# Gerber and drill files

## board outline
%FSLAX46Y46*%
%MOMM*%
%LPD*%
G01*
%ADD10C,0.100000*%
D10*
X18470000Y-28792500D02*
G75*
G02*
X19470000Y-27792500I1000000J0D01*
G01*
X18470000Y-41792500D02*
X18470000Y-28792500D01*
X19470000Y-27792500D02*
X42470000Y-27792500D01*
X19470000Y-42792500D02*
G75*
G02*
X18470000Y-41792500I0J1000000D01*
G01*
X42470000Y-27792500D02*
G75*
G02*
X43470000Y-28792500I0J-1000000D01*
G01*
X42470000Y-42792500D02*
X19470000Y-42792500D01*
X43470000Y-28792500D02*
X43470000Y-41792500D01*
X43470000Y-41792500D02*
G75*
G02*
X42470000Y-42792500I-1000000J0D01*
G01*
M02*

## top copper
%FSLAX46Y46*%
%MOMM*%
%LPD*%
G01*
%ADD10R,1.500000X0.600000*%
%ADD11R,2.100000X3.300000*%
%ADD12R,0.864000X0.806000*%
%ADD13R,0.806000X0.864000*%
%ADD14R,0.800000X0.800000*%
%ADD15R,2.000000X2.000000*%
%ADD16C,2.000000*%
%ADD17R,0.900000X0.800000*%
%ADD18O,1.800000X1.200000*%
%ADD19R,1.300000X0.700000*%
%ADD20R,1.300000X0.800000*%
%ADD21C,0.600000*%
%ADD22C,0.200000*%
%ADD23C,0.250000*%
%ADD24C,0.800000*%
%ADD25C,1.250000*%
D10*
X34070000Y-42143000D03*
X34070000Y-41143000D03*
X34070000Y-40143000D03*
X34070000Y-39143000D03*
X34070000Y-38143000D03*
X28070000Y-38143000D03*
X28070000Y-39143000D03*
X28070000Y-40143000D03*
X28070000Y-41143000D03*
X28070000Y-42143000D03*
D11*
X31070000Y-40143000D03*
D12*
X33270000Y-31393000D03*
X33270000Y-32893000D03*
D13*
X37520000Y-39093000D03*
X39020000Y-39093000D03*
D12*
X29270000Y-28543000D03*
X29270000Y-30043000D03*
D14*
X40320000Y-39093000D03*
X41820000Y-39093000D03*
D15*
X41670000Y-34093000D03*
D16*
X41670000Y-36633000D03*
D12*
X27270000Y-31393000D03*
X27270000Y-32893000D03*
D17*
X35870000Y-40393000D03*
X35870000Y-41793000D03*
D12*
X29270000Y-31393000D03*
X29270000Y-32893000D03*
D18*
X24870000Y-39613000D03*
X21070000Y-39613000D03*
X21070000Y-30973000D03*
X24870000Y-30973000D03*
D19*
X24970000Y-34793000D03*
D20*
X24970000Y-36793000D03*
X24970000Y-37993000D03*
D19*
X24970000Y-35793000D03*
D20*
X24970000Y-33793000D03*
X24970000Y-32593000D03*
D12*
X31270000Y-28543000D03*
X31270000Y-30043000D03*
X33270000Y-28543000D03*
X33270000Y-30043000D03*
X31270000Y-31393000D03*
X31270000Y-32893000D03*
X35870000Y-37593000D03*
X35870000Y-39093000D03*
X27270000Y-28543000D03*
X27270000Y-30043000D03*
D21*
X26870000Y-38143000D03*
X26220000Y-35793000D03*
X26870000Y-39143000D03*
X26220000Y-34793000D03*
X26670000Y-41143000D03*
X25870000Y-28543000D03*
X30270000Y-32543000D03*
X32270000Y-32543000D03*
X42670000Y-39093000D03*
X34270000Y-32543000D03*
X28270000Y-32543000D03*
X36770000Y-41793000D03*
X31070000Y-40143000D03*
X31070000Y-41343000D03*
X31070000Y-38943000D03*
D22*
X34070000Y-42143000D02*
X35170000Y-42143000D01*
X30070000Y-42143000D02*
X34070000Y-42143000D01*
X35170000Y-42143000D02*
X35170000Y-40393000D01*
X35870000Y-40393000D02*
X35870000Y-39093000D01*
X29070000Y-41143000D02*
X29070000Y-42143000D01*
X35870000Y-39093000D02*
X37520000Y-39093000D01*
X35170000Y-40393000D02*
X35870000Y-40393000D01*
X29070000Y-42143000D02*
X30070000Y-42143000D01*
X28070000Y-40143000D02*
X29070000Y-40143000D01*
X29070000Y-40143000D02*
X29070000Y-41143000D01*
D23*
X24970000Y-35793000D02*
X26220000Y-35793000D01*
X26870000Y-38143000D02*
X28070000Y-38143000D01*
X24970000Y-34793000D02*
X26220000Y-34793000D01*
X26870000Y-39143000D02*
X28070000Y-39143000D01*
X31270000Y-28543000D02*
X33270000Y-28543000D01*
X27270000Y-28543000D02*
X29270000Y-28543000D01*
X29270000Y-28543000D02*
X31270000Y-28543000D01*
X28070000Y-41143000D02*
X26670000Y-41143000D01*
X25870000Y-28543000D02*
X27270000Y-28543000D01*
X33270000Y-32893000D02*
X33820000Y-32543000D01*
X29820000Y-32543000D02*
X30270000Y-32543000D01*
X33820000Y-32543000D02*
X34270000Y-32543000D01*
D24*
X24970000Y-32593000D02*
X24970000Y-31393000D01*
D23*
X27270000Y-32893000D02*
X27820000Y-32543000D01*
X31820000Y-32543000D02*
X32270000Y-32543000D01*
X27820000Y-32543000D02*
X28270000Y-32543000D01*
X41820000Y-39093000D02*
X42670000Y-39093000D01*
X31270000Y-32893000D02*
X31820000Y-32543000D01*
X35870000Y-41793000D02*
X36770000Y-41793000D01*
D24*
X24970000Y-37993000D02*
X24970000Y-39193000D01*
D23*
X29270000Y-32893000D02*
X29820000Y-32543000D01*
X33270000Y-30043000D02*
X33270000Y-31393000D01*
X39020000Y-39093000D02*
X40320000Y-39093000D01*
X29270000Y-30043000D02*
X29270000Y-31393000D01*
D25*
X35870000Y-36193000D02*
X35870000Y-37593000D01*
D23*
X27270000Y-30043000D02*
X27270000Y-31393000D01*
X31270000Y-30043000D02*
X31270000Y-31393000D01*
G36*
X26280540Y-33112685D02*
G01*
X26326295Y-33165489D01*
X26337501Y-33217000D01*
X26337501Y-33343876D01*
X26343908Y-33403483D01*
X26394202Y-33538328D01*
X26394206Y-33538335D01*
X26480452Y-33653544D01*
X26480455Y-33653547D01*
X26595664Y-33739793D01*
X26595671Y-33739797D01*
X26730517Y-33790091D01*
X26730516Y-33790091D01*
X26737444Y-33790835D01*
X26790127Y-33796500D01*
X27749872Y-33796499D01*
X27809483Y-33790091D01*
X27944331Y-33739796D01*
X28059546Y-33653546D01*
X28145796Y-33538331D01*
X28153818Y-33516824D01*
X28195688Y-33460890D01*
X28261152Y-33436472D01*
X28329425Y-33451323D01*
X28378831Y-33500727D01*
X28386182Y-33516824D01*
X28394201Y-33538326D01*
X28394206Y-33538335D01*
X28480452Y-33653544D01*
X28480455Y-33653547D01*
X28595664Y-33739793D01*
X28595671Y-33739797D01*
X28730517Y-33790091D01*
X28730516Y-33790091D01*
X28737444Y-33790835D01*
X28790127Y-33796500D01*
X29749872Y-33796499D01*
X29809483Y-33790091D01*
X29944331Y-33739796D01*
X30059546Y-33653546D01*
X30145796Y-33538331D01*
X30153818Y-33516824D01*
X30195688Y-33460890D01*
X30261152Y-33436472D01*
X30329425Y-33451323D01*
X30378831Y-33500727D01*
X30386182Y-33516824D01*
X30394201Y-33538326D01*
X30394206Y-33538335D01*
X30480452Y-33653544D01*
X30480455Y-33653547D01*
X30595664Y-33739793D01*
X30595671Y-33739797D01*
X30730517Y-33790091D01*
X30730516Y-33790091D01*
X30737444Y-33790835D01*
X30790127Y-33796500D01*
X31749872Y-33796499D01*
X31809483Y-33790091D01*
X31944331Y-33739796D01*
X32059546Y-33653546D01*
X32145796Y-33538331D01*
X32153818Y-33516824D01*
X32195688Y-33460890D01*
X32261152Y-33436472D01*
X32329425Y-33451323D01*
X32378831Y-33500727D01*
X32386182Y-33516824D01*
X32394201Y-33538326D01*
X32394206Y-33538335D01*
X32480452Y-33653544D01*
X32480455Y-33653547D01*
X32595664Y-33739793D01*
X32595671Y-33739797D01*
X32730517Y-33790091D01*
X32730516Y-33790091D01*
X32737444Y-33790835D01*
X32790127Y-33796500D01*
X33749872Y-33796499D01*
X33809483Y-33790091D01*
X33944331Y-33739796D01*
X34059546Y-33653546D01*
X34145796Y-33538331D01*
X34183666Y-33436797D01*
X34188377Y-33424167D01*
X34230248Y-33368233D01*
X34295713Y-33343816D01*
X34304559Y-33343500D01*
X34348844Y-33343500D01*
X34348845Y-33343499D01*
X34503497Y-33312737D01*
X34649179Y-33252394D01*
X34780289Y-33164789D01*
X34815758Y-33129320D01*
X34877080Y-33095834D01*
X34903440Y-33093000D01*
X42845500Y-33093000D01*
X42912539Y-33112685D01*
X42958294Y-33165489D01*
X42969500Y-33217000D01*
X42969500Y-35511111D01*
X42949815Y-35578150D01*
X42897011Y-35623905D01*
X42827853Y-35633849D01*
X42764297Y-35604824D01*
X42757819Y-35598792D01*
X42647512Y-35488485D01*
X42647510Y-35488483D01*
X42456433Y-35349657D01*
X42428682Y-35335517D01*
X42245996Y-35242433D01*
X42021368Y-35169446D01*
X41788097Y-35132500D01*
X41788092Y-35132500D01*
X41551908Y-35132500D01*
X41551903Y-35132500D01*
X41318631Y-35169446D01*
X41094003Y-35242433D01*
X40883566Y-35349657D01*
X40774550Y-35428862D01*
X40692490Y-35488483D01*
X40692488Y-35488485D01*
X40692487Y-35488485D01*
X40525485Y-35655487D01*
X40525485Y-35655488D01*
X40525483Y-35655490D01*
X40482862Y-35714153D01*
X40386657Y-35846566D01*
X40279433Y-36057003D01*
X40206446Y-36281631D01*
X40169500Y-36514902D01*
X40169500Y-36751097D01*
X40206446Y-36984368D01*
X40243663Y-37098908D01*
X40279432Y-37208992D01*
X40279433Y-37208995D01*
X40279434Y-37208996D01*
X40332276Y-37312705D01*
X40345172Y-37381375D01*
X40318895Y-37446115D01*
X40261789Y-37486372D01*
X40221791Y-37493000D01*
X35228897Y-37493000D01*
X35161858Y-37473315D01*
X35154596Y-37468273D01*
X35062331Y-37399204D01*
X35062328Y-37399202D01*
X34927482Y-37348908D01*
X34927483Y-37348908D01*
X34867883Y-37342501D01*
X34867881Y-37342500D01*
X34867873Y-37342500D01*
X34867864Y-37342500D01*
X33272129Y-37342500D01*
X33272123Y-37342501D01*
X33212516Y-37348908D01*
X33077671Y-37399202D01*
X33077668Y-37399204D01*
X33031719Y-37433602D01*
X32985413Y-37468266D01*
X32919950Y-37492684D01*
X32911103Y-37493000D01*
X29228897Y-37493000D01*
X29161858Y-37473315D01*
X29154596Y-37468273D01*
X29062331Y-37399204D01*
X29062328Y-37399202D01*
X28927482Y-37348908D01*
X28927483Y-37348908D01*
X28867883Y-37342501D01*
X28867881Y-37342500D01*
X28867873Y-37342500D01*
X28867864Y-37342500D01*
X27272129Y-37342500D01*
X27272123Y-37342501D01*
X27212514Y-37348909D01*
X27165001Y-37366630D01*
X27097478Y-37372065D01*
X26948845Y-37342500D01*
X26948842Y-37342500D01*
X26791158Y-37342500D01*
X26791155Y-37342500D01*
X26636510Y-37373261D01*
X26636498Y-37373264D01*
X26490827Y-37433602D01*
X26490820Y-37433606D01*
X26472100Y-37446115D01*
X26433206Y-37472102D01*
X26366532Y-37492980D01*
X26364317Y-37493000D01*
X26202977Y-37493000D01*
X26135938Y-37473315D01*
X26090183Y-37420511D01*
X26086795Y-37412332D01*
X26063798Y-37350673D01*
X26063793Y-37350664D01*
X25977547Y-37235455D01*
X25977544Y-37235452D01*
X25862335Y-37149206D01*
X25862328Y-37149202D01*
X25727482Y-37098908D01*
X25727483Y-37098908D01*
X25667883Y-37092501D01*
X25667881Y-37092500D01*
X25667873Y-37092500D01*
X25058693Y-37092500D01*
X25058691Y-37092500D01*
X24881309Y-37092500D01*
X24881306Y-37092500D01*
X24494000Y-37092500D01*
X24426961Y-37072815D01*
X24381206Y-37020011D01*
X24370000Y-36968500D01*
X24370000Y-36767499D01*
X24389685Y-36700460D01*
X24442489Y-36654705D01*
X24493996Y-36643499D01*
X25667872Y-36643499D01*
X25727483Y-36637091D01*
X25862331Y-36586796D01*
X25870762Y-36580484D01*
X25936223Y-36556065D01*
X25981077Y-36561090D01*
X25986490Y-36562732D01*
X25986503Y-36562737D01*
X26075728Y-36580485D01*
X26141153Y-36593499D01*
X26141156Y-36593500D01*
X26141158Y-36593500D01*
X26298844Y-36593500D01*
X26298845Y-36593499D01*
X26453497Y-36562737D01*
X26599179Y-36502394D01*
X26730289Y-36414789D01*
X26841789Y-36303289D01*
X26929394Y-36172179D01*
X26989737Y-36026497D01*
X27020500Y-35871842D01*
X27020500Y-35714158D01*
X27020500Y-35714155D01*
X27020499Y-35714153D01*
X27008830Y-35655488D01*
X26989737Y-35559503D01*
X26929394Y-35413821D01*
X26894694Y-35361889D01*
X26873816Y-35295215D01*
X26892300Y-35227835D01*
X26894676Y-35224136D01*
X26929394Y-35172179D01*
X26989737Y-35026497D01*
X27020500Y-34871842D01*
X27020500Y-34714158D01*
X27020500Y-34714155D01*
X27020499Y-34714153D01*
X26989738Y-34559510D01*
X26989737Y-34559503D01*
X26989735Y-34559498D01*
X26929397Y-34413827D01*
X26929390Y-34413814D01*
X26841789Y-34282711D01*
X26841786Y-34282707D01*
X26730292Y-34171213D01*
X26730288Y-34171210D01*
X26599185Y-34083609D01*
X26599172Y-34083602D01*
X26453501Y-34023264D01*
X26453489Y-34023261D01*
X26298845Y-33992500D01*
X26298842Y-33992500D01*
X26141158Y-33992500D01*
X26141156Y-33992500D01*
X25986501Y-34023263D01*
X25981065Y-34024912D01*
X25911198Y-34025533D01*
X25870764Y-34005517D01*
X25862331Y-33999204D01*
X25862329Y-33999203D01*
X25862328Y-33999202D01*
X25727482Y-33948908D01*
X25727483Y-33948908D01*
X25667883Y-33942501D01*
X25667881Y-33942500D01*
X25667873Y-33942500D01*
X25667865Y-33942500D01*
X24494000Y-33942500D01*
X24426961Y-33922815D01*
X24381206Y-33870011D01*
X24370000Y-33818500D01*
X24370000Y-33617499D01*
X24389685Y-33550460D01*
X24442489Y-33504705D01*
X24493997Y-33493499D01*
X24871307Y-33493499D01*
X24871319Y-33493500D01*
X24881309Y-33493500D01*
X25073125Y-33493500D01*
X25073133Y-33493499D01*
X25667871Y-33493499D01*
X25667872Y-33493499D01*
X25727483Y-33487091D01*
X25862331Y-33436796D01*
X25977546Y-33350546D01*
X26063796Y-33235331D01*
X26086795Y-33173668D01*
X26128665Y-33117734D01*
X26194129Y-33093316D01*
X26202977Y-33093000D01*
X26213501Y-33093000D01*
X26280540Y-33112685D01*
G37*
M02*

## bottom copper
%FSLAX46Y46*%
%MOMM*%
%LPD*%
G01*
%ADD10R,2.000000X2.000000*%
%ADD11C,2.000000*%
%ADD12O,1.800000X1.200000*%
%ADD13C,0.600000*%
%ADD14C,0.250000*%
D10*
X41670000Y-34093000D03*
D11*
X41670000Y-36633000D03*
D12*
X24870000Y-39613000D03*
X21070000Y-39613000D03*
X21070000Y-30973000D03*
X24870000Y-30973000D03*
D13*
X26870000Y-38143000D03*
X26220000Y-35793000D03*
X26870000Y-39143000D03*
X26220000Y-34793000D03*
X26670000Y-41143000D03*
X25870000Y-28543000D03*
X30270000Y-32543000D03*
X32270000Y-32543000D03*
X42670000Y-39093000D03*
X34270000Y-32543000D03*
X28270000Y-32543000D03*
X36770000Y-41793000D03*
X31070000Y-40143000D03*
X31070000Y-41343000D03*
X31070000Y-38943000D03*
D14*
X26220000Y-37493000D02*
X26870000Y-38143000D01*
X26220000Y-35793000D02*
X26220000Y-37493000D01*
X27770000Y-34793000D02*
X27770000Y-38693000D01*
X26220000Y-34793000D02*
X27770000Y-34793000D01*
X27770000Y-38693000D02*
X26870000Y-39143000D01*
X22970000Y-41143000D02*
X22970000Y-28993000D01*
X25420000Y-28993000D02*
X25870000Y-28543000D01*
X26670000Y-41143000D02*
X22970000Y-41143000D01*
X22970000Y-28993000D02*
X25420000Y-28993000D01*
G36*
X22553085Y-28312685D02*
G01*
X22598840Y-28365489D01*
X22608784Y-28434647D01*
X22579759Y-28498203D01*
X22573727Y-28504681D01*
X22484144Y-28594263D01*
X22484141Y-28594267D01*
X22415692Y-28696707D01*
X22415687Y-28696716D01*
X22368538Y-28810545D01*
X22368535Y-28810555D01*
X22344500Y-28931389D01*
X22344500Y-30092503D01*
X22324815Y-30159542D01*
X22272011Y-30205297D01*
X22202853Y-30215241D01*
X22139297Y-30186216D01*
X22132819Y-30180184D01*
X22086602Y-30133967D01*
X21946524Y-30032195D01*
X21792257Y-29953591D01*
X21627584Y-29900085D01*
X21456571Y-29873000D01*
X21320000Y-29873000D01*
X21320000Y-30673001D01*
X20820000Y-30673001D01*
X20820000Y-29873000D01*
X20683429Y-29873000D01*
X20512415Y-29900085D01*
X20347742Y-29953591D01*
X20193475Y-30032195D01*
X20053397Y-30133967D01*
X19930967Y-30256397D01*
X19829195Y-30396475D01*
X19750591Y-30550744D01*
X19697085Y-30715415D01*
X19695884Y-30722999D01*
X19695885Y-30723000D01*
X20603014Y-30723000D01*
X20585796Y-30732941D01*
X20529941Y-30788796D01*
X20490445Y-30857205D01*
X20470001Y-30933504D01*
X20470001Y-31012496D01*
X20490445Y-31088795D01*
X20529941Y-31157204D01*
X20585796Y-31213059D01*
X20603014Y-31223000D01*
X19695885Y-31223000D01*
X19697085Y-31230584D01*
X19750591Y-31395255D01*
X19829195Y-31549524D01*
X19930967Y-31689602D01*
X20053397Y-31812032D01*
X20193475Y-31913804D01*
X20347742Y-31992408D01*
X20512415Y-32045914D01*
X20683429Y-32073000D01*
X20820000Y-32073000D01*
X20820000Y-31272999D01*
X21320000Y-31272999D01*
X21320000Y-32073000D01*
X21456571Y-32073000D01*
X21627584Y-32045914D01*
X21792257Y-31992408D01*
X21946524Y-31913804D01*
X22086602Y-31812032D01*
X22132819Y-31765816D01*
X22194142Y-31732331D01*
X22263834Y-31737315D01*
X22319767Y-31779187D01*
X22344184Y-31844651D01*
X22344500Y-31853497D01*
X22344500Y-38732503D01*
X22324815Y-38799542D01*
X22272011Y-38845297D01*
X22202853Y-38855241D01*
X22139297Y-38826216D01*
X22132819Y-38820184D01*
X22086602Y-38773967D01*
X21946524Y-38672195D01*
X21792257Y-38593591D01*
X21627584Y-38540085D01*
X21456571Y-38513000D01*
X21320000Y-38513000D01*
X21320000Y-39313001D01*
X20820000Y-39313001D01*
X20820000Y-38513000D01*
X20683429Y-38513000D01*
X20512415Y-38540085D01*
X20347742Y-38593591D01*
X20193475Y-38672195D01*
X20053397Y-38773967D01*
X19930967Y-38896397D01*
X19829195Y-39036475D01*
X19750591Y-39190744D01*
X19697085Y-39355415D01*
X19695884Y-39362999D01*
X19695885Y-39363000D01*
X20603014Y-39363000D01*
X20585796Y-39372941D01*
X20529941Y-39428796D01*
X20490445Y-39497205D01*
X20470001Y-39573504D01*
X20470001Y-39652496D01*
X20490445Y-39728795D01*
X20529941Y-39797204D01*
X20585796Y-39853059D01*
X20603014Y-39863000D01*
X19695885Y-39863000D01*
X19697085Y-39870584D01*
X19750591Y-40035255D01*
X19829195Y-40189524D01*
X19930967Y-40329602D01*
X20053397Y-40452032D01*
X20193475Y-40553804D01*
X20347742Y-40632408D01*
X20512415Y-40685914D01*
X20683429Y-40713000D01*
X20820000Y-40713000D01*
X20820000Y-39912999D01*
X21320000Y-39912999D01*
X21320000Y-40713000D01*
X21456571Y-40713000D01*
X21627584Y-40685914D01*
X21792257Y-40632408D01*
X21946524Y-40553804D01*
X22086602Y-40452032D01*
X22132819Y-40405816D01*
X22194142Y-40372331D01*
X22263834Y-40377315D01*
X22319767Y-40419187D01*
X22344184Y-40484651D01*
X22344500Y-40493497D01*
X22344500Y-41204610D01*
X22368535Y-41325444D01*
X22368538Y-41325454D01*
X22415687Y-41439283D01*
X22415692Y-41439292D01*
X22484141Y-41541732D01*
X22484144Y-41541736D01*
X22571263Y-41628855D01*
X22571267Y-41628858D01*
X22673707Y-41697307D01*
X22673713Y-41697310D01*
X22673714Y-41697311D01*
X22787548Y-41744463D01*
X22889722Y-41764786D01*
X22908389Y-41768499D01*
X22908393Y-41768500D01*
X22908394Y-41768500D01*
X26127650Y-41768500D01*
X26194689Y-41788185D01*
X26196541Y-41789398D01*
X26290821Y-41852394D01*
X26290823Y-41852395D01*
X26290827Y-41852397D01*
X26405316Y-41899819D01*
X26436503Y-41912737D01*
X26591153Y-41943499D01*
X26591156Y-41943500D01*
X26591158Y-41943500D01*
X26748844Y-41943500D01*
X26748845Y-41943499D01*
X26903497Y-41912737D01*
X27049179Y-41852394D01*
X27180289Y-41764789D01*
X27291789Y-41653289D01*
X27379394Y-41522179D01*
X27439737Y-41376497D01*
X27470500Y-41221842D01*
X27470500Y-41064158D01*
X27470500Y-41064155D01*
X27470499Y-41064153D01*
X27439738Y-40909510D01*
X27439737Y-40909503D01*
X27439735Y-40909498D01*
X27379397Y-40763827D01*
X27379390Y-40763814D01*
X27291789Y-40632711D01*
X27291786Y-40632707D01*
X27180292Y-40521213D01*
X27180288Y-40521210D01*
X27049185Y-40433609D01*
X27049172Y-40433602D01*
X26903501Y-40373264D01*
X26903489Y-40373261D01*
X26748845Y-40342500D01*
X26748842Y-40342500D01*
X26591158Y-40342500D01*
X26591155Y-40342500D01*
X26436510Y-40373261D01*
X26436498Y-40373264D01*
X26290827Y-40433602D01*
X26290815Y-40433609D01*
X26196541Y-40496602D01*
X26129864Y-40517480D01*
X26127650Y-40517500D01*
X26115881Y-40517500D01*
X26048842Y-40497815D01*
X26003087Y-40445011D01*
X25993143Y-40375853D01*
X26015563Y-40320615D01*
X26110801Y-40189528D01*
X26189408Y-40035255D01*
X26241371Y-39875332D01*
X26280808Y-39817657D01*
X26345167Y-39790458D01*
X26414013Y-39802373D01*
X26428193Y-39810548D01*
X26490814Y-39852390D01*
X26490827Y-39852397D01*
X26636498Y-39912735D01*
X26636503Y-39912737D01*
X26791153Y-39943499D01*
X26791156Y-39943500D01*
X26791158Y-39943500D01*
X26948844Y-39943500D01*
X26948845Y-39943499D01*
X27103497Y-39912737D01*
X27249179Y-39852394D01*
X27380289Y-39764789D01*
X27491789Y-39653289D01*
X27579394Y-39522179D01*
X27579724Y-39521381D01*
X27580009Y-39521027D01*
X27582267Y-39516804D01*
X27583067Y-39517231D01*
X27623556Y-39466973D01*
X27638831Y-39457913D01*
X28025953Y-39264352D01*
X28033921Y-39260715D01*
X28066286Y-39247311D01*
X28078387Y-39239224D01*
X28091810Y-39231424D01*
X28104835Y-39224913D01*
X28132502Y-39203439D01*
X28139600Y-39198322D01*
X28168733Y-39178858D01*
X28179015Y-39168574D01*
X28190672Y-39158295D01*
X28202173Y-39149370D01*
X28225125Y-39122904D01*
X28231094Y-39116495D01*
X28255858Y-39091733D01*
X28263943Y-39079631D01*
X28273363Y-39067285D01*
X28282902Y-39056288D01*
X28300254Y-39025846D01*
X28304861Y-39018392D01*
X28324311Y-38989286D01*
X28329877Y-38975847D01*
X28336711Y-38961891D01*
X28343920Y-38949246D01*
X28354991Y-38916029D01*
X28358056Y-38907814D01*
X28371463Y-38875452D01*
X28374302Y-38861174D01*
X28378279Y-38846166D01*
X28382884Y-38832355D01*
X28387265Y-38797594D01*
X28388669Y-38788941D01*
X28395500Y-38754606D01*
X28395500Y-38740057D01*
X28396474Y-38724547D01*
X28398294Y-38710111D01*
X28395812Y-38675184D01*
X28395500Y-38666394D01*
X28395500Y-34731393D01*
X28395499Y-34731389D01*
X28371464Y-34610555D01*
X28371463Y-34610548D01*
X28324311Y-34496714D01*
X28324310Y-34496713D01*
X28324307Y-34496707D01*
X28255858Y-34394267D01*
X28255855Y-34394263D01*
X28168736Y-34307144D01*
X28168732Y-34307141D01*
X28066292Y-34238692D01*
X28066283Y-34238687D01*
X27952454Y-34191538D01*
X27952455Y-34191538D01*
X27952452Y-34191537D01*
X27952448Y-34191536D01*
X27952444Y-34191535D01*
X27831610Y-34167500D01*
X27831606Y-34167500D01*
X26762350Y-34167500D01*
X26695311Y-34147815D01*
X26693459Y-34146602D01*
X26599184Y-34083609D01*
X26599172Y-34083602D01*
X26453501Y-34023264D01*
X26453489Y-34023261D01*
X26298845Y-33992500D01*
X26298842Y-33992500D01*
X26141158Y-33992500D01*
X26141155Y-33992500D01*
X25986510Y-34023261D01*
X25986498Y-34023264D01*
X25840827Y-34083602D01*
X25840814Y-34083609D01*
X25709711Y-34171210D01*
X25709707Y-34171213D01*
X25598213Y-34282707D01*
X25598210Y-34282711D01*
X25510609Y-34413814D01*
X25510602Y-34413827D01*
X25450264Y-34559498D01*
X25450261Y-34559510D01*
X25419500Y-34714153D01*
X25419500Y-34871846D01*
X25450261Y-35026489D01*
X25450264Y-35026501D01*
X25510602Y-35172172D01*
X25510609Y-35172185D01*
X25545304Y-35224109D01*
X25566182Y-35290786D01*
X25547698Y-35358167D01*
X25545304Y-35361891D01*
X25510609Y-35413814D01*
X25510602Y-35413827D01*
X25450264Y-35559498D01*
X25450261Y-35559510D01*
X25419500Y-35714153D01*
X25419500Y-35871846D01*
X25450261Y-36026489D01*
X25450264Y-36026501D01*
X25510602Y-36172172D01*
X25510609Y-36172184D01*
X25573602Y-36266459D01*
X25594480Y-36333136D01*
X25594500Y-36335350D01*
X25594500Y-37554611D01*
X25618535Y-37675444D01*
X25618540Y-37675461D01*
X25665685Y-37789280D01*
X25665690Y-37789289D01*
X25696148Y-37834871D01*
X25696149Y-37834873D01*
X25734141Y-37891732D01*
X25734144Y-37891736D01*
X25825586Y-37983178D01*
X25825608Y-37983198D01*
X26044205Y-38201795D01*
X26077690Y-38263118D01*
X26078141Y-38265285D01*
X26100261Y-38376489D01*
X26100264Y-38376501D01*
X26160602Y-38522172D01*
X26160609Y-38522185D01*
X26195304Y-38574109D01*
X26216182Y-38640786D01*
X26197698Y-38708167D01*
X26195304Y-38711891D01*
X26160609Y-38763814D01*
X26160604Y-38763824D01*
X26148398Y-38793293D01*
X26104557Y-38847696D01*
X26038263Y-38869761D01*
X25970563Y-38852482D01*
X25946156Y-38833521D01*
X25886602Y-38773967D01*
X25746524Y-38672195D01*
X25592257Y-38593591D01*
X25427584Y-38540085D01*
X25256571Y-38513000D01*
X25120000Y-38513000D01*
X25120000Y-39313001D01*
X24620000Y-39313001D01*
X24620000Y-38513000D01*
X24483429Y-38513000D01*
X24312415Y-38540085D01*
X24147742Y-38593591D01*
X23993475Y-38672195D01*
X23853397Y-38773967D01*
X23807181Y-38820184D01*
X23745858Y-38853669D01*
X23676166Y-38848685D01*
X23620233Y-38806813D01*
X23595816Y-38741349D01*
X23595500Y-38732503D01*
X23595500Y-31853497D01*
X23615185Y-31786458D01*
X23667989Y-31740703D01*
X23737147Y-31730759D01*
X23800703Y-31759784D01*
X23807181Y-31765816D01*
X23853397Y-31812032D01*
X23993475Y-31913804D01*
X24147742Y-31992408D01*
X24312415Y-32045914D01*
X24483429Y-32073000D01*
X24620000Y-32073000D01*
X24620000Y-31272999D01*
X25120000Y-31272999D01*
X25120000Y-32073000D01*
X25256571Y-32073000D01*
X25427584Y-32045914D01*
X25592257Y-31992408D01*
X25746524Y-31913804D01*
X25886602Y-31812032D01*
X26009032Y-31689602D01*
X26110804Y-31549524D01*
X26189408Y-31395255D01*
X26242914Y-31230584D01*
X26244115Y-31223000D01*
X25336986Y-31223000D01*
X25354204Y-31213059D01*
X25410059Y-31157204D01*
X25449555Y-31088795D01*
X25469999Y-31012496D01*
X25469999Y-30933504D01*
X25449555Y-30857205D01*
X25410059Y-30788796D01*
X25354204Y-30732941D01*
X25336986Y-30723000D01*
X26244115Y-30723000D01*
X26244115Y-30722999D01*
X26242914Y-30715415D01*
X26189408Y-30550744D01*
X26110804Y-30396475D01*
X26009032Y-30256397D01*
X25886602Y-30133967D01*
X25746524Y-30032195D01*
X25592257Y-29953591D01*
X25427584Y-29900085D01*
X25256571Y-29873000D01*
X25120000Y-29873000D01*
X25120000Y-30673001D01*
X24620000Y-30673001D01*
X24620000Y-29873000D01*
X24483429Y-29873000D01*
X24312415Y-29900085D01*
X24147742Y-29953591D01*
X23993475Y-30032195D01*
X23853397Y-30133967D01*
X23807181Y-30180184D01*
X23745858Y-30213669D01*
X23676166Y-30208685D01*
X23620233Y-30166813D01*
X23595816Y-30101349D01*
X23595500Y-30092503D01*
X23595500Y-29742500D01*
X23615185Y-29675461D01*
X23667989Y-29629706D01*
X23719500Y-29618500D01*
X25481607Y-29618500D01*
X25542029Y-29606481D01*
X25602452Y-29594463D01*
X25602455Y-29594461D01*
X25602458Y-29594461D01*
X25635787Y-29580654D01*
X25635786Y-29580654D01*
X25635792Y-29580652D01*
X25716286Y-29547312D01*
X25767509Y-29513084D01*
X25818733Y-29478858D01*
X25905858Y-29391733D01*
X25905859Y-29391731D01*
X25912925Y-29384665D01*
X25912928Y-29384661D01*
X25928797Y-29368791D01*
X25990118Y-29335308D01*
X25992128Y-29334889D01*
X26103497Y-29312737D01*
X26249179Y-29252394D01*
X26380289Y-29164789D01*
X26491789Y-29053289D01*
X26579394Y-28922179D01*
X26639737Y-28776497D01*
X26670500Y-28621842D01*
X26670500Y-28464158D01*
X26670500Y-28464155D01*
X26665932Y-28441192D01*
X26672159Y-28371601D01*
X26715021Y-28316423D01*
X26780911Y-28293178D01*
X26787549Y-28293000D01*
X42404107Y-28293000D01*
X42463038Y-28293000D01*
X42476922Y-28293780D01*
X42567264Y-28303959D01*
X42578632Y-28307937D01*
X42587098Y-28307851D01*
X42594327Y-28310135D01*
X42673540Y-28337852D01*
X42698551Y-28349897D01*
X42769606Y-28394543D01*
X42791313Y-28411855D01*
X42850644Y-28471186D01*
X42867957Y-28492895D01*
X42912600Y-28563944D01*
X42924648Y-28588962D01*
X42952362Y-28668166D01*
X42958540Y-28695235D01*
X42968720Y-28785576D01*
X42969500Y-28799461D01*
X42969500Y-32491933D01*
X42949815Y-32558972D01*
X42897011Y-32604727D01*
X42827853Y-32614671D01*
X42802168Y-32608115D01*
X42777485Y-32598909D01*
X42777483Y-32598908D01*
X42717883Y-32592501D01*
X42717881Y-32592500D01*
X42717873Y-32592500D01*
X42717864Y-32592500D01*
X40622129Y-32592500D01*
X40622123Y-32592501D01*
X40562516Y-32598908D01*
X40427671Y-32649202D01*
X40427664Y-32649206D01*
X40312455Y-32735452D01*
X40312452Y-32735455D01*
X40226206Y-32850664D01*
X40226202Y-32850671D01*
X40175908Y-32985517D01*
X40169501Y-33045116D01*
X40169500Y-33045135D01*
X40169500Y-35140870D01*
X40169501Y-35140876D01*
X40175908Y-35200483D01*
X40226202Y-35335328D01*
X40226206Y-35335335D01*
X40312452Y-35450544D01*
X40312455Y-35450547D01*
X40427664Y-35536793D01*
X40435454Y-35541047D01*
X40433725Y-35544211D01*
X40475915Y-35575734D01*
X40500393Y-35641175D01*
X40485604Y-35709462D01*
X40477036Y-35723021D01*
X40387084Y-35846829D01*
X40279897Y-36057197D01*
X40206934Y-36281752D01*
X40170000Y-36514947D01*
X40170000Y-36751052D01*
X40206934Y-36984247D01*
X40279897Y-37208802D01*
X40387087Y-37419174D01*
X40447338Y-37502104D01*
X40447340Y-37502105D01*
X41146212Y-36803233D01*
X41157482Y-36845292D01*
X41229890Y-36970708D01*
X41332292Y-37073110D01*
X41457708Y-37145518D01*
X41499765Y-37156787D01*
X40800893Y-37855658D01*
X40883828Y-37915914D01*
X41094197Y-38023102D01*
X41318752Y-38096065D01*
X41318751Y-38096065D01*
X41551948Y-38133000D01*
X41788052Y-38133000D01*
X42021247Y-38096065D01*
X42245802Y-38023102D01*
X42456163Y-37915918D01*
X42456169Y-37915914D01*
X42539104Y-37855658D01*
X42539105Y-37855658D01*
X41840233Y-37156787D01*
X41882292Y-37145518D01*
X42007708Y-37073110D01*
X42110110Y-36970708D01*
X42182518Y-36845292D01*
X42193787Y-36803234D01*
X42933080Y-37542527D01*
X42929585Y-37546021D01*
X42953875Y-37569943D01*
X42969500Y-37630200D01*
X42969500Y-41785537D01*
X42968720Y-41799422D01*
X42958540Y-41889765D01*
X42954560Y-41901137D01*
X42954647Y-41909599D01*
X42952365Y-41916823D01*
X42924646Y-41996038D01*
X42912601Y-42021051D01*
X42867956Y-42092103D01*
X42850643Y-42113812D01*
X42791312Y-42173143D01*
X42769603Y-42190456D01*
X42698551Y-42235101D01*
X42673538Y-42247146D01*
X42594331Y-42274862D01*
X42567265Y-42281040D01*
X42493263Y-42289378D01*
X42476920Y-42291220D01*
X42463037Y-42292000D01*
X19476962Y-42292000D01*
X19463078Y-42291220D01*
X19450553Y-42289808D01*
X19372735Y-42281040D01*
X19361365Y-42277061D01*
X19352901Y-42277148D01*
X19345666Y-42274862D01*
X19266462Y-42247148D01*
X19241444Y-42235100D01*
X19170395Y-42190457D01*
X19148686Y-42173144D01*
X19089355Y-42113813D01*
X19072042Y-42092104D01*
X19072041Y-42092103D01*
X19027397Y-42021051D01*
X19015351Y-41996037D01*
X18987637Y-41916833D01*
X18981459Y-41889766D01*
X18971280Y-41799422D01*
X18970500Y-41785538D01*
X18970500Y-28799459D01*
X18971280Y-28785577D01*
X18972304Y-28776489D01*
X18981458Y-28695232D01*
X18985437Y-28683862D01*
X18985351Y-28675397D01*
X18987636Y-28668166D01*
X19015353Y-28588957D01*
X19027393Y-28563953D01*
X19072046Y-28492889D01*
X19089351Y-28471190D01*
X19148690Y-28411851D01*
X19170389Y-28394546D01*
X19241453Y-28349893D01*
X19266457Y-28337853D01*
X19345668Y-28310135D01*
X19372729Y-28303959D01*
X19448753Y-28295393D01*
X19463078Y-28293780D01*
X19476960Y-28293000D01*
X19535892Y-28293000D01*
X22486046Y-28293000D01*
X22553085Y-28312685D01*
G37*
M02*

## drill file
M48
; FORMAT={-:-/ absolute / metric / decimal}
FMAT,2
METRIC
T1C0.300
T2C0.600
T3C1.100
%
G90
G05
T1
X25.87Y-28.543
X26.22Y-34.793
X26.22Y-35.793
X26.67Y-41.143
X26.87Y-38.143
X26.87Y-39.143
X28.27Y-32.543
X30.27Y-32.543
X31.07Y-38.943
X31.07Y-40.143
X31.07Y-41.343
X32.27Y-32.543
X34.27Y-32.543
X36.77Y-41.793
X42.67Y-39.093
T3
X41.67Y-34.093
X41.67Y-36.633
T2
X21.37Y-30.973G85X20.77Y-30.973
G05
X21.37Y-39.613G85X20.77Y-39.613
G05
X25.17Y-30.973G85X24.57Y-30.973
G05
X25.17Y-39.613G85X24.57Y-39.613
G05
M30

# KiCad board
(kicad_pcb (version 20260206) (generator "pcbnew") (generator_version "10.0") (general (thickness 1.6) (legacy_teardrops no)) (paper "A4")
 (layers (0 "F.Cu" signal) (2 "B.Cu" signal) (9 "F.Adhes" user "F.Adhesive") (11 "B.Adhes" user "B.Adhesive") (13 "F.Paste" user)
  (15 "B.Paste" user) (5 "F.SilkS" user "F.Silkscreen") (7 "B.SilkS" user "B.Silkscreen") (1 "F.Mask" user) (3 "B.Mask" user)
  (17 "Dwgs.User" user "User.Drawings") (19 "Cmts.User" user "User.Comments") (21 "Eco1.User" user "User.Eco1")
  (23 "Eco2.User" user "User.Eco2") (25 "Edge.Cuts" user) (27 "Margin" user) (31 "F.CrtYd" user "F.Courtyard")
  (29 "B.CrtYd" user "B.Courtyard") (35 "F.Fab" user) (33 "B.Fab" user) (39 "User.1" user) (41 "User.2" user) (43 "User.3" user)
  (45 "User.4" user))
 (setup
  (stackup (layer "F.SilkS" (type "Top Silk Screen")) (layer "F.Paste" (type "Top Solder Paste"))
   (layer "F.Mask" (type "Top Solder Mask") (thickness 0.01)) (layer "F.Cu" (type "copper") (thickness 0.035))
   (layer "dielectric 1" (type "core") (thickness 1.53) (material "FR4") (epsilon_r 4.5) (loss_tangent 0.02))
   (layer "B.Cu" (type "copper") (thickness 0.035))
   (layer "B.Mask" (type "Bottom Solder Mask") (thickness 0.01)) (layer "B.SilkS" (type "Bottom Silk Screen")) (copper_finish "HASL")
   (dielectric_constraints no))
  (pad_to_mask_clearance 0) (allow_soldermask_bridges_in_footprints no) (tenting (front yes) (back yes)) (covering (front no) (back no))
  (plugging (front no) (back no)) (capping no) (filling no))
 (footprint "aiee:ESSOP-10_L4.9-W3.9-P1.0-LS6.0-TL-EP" (layer "F.Cu") (at 31.07 40.143 90)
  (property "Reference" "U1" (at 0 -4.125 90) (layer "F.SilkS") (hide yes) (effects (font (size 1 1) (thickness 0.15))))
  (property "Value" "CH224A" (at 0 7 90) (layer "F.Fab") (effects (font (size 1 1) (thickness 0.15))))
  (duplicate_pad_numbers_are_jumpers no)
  (pad "1" smd rect (at -2 3 180) (size 1.5 0.6) (layers "F.Cu" "F.Mask" "F.Paste") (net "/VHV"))
  (pad "2" smd rect (at -1 3 180) (size 1.5 0.6) (layers "F.Cu" "F.Mask" "F.Paste") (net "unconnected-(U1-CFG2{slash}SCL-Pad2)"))
  (pad "3" smd rect (at 0 3 180) (size 1.5 0.6) (layers "F.Cu" "F.Mask" "F.Paste") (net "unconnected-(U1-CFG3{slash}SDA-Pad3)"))
  (pad "4" smd rect (at 1 3 180) (size 1.5 0.6) (layers "F.Cu" "F.Mask" "F.Paste") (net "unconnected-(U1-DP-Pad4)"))
  (pad "5" smd rect (at 2 3 180) (size 1.5 0.6) (layers "F.Cu" "F.Mask" "F.Paste") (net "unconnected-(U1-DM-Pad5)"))
  (pad "6" smd rect (at 2 -3 180) (size 1.5 0.6) (layers "F.Cu" "F.Mask" "F.Paste") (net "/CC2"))
  (pad "7" smd rect (at 1 -3 180) (size 1.5 0.6) (layers "F.Cu" "F.Mask" "F.Paste") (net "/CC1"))
  (pad "8" smd rect (at 0 -3 180) (size 1.5 0.6) (layers "F.Cu" "F.Mask" "F.Paste") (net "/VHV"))
  (pad "9" smd rect (at -1 -3 180) (size 1.5 0.6) (layers "F.Cu" "F.Mask" "F.Paste") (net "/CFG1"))
  (pad "10" smd rect (at -2 -3 180) (size 1.5 0.6) (layers "F.Cu" "F.Mask" "F.Paste") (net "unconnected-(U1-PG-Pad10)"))
  (pad "11" smd rect (at 0 0 270) (size 3.3 2.1) (layers "F.Cu" "F.Mask" "F.Paste") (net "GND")))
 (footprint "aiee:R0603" (layer "F.Cu") (at 33.27 32.143 -90)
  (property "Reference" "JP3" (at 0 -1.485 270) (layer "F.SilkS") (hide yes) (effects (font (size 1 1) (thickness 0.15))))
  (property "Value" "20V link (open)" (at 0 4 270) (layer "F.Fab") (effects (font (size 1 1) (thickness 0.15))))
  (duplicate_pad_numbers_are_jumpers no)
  (pad "1" smd rect (at -0.75 0 270) (size 0.806 0.864) (layers "F.Cu" "F.Mask" "F.Paste") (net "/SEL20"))
  (pad "2" smd rect (at 0.75 0 270) (size 0.806 0.864) (layers "F.Cu" "F.Mask" "F.Paste") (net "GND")))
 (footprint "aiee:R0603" (layer "F.Cu") (at 38.27 39.093)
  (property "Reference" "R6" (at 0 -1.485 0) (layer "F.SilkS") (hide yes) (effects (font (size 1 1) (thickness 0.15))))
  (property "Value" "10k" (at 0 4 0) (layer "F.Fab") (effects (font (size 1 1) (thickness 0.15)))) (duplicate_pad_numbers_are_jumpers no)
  (pad "1" smd rect (at -0.75 0) (size 0.806 0.864) (layers "F.Cu" "F.Mask" "F.Paste") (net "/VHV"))
  (pad "2" smd rect (at 0.75 0) (size 0.806 0.864) (layers "F.Cu" "F.Mask" "F.Paste") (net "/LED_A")))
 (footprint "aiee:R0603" (layer "F.Cu") (at 29.27 29.293 -90)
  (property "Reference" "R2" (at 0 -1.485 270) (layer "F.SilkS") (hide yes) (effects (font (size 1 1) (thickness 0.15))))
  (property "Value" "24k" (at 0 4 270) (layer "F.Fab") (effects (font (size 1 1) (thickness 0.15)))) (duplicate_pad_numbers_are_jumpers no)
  (pad "1" smd rect (at -0.75 0 270) (size 0.806 0.864) (layers "F.Cu" "F.Mask" "F.Paste") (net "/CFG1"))
  (pad "2" smd rect (at 0.75 0 270) (size 0.806 0.864) (layers "F.Cu" "F.Mask" "F.Paste") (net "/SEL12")))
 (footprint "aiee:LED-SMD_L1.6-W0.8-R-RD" (layer "F.Cu") (at 41.07 39.093 180)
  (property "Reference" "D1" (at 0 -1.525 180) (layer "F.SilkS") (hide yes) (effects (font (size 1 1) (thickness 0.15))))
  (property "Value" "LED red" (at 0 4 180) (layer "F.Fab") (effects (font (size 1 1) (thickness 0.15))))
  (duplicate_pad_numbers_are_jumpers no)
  (pad "1" smd rect (at 0.75 0 180) (size 0.8 0.8) (layers "F.Cu" "F.Mask" "F.Paste") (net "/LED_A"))
  (pad "2" smd rect (at -0.75 0 180) (size 0.8 0.8) (layers "F.Cu" "F.Mask" "F.Paste") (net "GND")))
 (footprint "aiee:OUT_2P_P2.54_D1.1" (layer "F.Cu") (at 41.67 34.093)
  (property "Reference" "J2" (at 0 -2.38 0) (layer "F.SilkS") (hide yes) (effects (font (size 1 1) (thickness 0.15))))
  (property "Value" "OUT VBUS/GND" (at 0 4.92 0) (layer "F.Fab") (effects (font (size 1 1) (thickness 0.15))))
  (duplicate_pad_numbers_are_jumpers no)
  (pad "1" thru_hole rect (at 0 0) (size 2 2) (drill 1.1) (layers "*.Cu" "*.Mask") (remove_unused_layers no) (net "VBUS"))
  (pad "2" thru_hole circle (at 0 2.54) (size 2 2) (drill 1.1) (layers "*.Cu" "*.Mask") (remove_unused_layers no) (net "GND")))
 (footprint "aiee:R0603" (layer "F.Cu") (at 27.27 32.143 -90)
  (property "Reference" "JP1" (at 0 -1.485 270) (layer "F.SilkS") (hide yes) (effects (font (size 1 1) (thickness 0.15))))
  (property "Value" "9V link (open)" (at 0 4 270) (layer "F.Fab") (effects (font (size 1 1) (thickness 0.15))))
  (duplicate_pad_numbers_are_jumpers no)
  (pad "1" smd rect (at -0.75 0 270) (size 0.806 0.864) (layers "F.Cu" "F.Mask" "F.Paste") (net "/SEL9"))
  (pad "2" smd rect (at 0.75 0 270) (size 0.806 0.864) (layers "F.Cu" "F.Mask" "F.Paste") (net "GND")))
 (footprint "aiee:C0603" (layer "F.Cu") (at 35.87 41.093 -90)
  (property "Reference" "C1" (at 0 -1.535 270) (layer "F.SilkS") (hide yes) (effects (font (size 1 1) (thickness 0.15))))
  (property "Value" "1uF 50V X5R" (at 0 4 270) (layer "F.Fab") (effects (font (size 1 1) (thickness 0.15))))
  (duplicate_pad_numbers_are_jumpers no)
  (pad "1" smd rect (at -0.7 0 270) (size 0.8 0.9) (layers "F.Cu" "F.Mask" "F.Paste") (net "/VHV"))
  (pad "2" smd rect (at 0.7 0 270) (size 0.8 0.9) (layers "F.Cu" "F.Mask" "F.Paste") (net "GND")))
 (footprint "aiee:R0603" (layer "F.Cu") (at 29.27 32.143 -90)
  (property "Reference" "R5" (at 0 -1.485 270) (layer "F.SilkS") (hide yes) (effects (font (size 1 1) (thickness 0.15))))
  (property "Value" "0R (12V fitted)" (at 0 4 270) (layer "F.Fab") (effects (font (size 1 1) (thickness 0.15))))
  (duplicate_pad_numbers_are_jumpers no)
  (pad "1" smd rect (at -0.75 0 270) (size 0.806 0.864) (layers "F.Cu" "F.Mask" "F.Paste") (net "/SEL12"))
  (pad "2" smd rect (at 0.75 0 270) (size 0.806 0.864) (layers "F.Cu" "F.Mask" "F.Paste") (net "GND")))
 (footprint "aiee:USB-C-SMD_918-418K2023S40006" (layer "F.Cu") (at 23.02 35.293 -90)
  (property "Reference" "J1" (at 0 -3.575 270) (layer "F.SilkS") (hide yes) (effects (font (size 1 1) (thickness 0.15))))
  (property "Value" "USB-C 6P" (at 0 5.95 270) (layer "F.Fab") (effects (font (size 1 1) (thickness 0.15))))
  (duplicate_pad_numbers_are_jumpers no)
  (pad "1" thru_hole oval (at 4.32 -1.85 270) (size 1.2 1.8) (drill oval 0.599998 1.199998) (layers "*.Cu" "*.Mask")
   (remove_unused_layers no) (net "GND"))
  (pad "2" thru_hole oval (at 4.32 1.95 270) (size 1.2 1.8) (drill oval 0.599998 1.199998) (layers "*.Cu" "*.Mask")
   (remove_unused_layers no) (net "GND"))
  (pad "3" thru_hole oval (at -4.32 1.95 270) (size 1.2 1.8) (drill oval 0.599998 1.199998) (layers "*.Cu" "*.Mask")
   (remove_unused_layers no) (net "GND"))
  (pad "4" thru_hole oval (at -4.32 -1.85 270) (size 1.2 1.8) (drill oval 0.599998 1.199998) (layers "*.Cu" "*.Mask")
   (remove_unused_layers no) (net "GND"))
  (pad "A5" smd rect (at -0.5 -1.95 270) (size 0.7 1.3) (layers "F.Cu" "F.Mask" "F.Paste") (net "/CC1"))
  (pad "A9" smd rect (at 1.5 -1.95 270) (size 0.8 1.3) (layers "F.Cu" "F.Mask" "F.Paste") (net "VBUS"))
  (pad "A12" smd rect (at 2.7 -1.95 270) (size 0.8 1.3) (layers "F.Cu" "F.Mask" "F.Paste") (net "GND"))
  (pad "B5" smd rect (at 0.5 -1.95 270) (size 0.7 1.3) (layers "F.Cu" "F.Mask" "F.Paste") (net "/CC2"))
  (pad "B9" smd rect (at -1.5 -1.95 270) (size 0.8 1.3) (layers "F.Cu" "F.Mask" "F.Paste") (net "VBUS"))
  (pad "B12" smd rect (at -2.7 -1.95 270) (size 0.8 1.3) (layers "F.Cu" "F.Mask" "F.Paste") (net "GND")))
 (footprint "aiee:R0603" (layer "F.Cu") (at 31.27 29.293 -90)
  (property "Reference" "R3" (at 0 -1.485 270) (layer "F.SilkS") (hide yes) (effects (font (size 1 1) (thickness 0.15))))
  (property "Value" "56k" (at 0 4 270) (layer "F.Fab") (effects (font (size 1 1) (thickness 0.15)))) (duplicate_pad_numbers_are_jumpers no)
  (pad "1" smd rect (at -0.75 0 270) (size 0.806 0.864) (layers "F.Cu" "F.Mask" "F.Paste") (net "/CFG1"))
  (pad "2" smd rect (at 0.75 0 270) (size 0.806 0.864) (layers "F.Cu" "F.Mask" "F.Paste") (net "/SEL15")))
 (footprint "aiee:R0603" (layer "F.Cu") (at 33.27 29.293 -90)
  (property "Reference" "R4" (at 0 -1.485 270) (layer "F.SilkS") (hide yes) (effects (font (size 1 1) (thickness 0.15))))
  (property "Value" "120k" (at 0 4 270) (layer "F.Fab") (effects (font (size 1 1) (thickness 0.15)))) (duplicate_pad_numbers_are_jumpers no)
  (pad "1" smd rect (at -0.75 0 270) (size 0.806 0.864) (layers "F.Cu" "F.Mask" "F.Paste") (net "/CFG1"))
  (pad "2" smd rect (at 0.75 0 270) (size 0.806 0.864) (layers "F.Cu" "F.Mask" "F.Paste") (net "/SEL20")))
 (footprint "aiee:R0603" (layer "F.Cu") (at 31.27 32.143 -90)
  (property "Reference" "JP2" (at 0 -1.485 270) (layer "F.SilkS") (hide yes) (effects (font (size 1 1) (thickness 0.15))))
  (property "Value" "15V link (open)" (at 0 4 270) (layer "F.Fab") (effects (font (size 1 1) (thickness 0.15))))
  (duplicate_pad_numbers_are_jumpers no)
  (pad "1" smd rect (at -0.75 0 270) (size 0.806 0.864) (layers "F.Cu" "F.Mask" "F.Paste") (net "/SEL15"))
  (pad "2" smd rect (at 0.75 0 270) (size 0.806 0.864) (layers "F.Cu" "F.Mask" "F.Paste") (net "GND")))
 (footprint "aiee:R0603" (layer "F.Cu") (at 35.87 38.343 -90)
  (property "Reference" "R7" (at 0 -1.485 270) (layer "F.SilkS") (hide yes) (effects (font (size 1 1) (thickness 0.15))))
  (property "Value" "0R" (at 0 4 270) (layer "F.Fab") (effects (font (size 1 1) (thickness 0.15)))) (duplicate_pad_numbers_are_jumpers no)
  (pad "1" smd rect (at -0.75 0 270) (size 0.806 0.864) (layers "F.Cu" "F.Mask" "F.Paste") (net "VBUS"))
  (pad "2" smd rect (at 0.75 0 270) (size 0.806 0.864) (layers "F.Cu" "F.Mask" "F.Paste") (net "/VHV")))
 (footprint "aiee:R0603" (layer "F.Cu") (at 27.27 29.293 -90)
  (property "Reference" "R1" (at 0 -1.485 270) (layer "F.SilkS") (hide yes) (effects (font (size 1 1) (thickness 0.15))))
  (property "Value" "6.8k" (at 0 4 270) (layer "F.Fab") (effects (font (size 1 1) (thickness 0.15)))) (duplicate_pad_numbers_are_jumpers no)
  (pad "1" smd rect (at -0.75 0 270) (size 0.806 0.864) (layers "F.Cu" "F.Mask" "F.Paste") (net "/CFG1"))
  (pad "2" smd rect (at 0.75 0 270) (size 0.806 0.864) (layers "F.Cu" "F.Mask" "F.Paste") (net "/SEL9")))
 (gr_arc (start 18.47 28.7925) (mid 18.762893 28.085393) (end 19.47 27.7925) (stroke (width 0.1) (type default)) (layer "Edge.Cuts"))
 (gr_line (start 18.47 41.7925) (end 18.47 28.7925) (stroke (width 0.1) (type default)) (layer "Edge.Cuts"))
 (gr_line (start 19.47 27.7925) (end 42.47 27.7925) (stroke (width 0.1) (type default)) (layer "Edge.Cuts"))
 (gr_arc (start 19.47 42.7925) (mid 18.762893 42.499606) (end 18.47 41.7925) (stroke (width 0.1) (type default)) (layer "Edge.Cuts"))
 (gr_arc (start 42.47 27.7925) (mid 43.177106 28.085393) (end 43.47 28.7925) (stroke (width 0.1) (type default)) (layer "Edge.Cuts"))
 (gr_line (start 42.47 42.7925) (end 19.47 42.7925) (stroke (width 0.1) (type default)) (layer "Edge.Cuts"))
 (gr_line (start 43.47 28.7925) (end 43.47 41.7925) (stroke (width 0.1) (type default)) (layer "Edge.Cuts"))
 (gr_arc (start 43.47 41.7925) (mid 43.177106 42.499606) (end 42.47 42.7925) (stroke (width 0.1) (type default)) (layer "Edge.Cuts"))
 (segment (start 34.07 42.143) (end 35.17 42.143) (width 0.2) (layer "F.Cu") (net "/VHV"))
 (segment (start 30.07 42.143) (end 34.07 42.143) (width 0.2) (layer "F.Cu") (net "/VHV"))
 (segment (start 35.17 42.143) (end 35.17 40.393) (width 0.2) (layer "F.Cu") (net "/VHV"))
 (segment (start 35.87 40.393) (end 35.87 39.093) (width 0.2) (layer "F.Cu") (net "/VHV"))
 (segment (start 29.07 41.143) (end 29.07 42.143) (width 0.2) (layer "F.Cu") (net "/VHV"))
 (segment (start 35.87 39.093) (end 37.52 39.093) (width 0.2) (layer "F.Cu") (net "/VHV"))
 (segment (start 35.17 40.393) (end 35.87 40.393) (width 0.2) (layer "F.Cu") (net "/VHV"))
 (segment (start 29.07 42.143) (end 30.07 42.143) (width 0.2) (layer "F.Cu") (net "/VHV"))
 (segment (start 28.07 40.143) (end 29.07 40.143) (width 0.2) (layer "F.Cu") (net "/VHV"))
 (segment (start 29.07 40.143) (end 29.07 41.143) (width 0.2) (layer "F.Cu") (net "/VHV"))
 (segment (start 24.97 35.793) (end 26.22 35.793) (width 0.25) (layer "F.Cu") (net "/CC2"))
 (segment (start 26.87 38.143) (end 28.07 38.143) (width 0.25) (layer "F.Cu") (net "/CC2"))
 (via (at 26.87 38.143) (size 0.6) (drill 0.3) (layers "F.Cu" "B.Cu") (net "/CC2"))
 (via (at 26.22 35.793) (size 0.6) (drill 0.3) (layers "F.Cu" "B.Cu") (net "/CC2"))
 (segment (start 26.22 37.493) (end 26.87 38.143) (width 0.25) (layer "B.Cu") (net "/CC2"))
 (segment (start 26.22 35.793) (end 26.22 37.493) (width 0.25) (layer "B.Cu") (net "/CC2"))
 (segment (start 24.97 34.793) (end 26.22 34.793) (width 0.25) (layer "F.Cu") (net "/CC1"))
 (segment (start 26.87 39.143) (end 28.07 39.143) (width 0.25) (layer "F.Cu") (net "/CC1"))
 (via (at 26.87 39.143) (size 0.6) (drill 0.3) (layers "F.Cu" "B.Cu") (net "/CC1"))
 (via (at 26.22 34.793) (size 0.6) (drill 0.3) (layers "F.Cu" "B.Cu") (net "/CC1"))
 (segment (start 27.77 34.793) (end 27.77 38.693) (width 0.25) (layer "B.Cu") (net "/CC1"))
 (segment (start 26.22 34.793) (end 27.77 34.793) (width 0.25) (layer "B.Cu") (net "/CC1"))
 (segment (start 27.77 38.693) (end 26.87 39.143) (width 0.25) (layer "B.Cu") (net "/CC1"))
 (segment (start 31.27 28.543) (end 33.27 28.543) (width 0.25) (layer "F.Cu") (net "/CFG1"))
 (segment (start 27.27 28.543) (end 29.27 28.543) (width 0.25) (layer "F.Cu") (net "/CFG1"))
 (segment (start 29.27 28.543) (end 31.27 28.543) (width 0.25) (layer "F.Cu") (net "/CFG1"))
 (segment (start 28.07 41.143) (end 26.67 41.143) (width 0.25) (layer "F.Cu") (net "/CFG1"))
 (segment (start 25.87 28.543) (end 27.27 28.543) (width 0.25) (layer "F.Cu") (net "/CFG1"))
 (via (at 26.67 41.143) (size 0.6) (drill 0.3) (layers "F.Cu" "B.Cu") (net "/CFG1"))
 (via (at 25.87 28.543) (size 0.6) (drill 0.3) (layers "F.Cu" "B.Cu") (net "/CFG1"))
 (segment (start 22.97 41.143) (end 22.97 28.993) (width 0.25) (layer "B.Cu") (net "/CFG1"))
 (segment (start 25.42 28.993) (end 25.87 28.543) (width 0.25) (layer "B.Cu") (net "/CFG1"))
 (segment (start 26.67 41.143) (end 22.97 41.143) (width 0.25) (layer "B.Cu") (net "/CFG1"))
 (segment (start 22.97 28.993) (end 25.42 28.993) (width 0.25) (layer "B.Cu") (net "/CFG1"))
 (segment (start 33.27 32.893) (end 33.82 32.543) (width 0.25) (layer "F.Cu") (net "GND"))
 (segment (start 29.82 32.543) (end 30.27 32.543) (width 0.25) (layer "F.Cu") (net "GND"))
 (segment (start 33.82 32.543) (end 34.27 32.543) (width 0.25) (layer "F.Cu") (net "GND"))
 (segment (start 24.97 32.593) (end 24.97 31.393) (width 0.8) (layer "F.Cu") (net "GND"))
 (segment (start 27.27 32.893) (end 27.82 32.543) (width 0.25) (layer "F.Cu") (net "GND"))
 (segment (start 31.82 32.543) (end 32.27 32.543) (width 0.25) (layer "F.Cu") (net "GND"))
 (segment (start 27.82 32.543) (end 28.27 32.543) (width 0.25) (layer "F.Cu") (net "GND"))
 (segment (start 41.82 39.093) (end 42.67 39.093) (width 0.25) (layer "F.Cu") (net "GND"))
 (segment (start 31.27 32.893) (end 31.82 32.543) (width 0.25) (layer "F.Cu") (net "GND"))
 (segment (start 35.87 41.793) (end 36.77 41.793) (width 0.25) (layer "F.Cu") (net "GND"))
 (segment (start 24.97 37.993) (end 24.97 39.193) (width 0.8) (layer "F.Cu") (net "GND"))
 (segment (start 29.27 32.893) (end 29.82 32.543) (width 0.25) (layer "F.Cu") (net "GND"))
 (via (at 30.27 32.543) (size 0.6) (drill 0.3) (layers "F.Cu" "B.Cu") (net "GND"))
 (via (at 32.27 32.543) (size 0.6) (drill 0.3) (layers "F.Cu" "B.Cu") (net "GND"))
 (via (at 42.67 39.093) (size 0.6) (drill 0.3) (layers "F.Cu" "B.Cu") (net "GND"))
 (via (at 34.27 32.543) (size 0.6) (drill 0.3) (layers "F.Cu" "B.Cu") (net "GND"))
 (via (at 28.27 32.543) (size 0.6) (drill 0.3) (layers "F.Cu" "B.Cu") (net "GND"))
 (via (at 36.77 41.793) (size 0.6) (drill 0.3) (layers "F.Cu" "B.Cu") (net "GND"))
 (via (at 31.07 40.143) (size 0.6) (drill 0.3) (layers "F.Cu" "B.Cu") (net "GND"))
 (via (at 31.07 41.343) (size 0.6) (drill 0.3) (layers "F.Cu" "B.Cu") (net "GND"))
 (via (at 31.07 38.943) (size 0.6) (drill 0.3) (layers "F.Cu" "B.Cu") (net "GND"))
 (segment (start 33.27 30.043) (end 33.27 31.393) (width 0.25) (layer "F.Cu") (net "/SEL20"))
 (segment (start 39.02 39.093) (end 40.32 39.093) (width 0.25) (layer "F.Cu") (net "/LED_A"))
 (segment (start 29.27 30.043) (end 29.27 31.393) (width 0.25) (layer "F.Cu") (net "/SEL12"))
 (segment (start 35.87 36.193) (end 35.87 37.593) (width 1.25) (layer "F.Cu") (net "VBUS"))
 (segment (start 27.27 30.043) (end 27.27 31.393) (width 0.25) (layer "F.Cu") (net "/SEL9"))
 (segment (start 31.27 30.043) (end 31.27 31.393) (width 0.25) (layer "F.Cu") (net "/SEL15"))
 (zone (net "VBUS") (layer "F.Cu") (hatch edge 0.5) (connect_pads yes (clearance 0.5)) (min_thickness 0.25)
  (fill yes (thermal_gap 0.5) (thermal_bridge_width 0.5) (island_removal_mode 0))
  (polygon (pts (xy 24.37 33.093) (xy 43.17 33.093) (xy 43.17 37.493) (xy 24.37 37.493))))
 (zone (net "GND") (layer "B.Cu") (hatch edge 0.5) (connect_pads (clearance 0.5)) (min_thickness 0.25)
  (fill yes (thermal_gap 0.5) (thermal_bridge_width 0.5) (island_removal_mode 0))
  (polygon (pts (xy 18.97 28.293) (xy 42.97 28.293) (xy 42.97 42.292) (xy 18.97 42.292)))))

